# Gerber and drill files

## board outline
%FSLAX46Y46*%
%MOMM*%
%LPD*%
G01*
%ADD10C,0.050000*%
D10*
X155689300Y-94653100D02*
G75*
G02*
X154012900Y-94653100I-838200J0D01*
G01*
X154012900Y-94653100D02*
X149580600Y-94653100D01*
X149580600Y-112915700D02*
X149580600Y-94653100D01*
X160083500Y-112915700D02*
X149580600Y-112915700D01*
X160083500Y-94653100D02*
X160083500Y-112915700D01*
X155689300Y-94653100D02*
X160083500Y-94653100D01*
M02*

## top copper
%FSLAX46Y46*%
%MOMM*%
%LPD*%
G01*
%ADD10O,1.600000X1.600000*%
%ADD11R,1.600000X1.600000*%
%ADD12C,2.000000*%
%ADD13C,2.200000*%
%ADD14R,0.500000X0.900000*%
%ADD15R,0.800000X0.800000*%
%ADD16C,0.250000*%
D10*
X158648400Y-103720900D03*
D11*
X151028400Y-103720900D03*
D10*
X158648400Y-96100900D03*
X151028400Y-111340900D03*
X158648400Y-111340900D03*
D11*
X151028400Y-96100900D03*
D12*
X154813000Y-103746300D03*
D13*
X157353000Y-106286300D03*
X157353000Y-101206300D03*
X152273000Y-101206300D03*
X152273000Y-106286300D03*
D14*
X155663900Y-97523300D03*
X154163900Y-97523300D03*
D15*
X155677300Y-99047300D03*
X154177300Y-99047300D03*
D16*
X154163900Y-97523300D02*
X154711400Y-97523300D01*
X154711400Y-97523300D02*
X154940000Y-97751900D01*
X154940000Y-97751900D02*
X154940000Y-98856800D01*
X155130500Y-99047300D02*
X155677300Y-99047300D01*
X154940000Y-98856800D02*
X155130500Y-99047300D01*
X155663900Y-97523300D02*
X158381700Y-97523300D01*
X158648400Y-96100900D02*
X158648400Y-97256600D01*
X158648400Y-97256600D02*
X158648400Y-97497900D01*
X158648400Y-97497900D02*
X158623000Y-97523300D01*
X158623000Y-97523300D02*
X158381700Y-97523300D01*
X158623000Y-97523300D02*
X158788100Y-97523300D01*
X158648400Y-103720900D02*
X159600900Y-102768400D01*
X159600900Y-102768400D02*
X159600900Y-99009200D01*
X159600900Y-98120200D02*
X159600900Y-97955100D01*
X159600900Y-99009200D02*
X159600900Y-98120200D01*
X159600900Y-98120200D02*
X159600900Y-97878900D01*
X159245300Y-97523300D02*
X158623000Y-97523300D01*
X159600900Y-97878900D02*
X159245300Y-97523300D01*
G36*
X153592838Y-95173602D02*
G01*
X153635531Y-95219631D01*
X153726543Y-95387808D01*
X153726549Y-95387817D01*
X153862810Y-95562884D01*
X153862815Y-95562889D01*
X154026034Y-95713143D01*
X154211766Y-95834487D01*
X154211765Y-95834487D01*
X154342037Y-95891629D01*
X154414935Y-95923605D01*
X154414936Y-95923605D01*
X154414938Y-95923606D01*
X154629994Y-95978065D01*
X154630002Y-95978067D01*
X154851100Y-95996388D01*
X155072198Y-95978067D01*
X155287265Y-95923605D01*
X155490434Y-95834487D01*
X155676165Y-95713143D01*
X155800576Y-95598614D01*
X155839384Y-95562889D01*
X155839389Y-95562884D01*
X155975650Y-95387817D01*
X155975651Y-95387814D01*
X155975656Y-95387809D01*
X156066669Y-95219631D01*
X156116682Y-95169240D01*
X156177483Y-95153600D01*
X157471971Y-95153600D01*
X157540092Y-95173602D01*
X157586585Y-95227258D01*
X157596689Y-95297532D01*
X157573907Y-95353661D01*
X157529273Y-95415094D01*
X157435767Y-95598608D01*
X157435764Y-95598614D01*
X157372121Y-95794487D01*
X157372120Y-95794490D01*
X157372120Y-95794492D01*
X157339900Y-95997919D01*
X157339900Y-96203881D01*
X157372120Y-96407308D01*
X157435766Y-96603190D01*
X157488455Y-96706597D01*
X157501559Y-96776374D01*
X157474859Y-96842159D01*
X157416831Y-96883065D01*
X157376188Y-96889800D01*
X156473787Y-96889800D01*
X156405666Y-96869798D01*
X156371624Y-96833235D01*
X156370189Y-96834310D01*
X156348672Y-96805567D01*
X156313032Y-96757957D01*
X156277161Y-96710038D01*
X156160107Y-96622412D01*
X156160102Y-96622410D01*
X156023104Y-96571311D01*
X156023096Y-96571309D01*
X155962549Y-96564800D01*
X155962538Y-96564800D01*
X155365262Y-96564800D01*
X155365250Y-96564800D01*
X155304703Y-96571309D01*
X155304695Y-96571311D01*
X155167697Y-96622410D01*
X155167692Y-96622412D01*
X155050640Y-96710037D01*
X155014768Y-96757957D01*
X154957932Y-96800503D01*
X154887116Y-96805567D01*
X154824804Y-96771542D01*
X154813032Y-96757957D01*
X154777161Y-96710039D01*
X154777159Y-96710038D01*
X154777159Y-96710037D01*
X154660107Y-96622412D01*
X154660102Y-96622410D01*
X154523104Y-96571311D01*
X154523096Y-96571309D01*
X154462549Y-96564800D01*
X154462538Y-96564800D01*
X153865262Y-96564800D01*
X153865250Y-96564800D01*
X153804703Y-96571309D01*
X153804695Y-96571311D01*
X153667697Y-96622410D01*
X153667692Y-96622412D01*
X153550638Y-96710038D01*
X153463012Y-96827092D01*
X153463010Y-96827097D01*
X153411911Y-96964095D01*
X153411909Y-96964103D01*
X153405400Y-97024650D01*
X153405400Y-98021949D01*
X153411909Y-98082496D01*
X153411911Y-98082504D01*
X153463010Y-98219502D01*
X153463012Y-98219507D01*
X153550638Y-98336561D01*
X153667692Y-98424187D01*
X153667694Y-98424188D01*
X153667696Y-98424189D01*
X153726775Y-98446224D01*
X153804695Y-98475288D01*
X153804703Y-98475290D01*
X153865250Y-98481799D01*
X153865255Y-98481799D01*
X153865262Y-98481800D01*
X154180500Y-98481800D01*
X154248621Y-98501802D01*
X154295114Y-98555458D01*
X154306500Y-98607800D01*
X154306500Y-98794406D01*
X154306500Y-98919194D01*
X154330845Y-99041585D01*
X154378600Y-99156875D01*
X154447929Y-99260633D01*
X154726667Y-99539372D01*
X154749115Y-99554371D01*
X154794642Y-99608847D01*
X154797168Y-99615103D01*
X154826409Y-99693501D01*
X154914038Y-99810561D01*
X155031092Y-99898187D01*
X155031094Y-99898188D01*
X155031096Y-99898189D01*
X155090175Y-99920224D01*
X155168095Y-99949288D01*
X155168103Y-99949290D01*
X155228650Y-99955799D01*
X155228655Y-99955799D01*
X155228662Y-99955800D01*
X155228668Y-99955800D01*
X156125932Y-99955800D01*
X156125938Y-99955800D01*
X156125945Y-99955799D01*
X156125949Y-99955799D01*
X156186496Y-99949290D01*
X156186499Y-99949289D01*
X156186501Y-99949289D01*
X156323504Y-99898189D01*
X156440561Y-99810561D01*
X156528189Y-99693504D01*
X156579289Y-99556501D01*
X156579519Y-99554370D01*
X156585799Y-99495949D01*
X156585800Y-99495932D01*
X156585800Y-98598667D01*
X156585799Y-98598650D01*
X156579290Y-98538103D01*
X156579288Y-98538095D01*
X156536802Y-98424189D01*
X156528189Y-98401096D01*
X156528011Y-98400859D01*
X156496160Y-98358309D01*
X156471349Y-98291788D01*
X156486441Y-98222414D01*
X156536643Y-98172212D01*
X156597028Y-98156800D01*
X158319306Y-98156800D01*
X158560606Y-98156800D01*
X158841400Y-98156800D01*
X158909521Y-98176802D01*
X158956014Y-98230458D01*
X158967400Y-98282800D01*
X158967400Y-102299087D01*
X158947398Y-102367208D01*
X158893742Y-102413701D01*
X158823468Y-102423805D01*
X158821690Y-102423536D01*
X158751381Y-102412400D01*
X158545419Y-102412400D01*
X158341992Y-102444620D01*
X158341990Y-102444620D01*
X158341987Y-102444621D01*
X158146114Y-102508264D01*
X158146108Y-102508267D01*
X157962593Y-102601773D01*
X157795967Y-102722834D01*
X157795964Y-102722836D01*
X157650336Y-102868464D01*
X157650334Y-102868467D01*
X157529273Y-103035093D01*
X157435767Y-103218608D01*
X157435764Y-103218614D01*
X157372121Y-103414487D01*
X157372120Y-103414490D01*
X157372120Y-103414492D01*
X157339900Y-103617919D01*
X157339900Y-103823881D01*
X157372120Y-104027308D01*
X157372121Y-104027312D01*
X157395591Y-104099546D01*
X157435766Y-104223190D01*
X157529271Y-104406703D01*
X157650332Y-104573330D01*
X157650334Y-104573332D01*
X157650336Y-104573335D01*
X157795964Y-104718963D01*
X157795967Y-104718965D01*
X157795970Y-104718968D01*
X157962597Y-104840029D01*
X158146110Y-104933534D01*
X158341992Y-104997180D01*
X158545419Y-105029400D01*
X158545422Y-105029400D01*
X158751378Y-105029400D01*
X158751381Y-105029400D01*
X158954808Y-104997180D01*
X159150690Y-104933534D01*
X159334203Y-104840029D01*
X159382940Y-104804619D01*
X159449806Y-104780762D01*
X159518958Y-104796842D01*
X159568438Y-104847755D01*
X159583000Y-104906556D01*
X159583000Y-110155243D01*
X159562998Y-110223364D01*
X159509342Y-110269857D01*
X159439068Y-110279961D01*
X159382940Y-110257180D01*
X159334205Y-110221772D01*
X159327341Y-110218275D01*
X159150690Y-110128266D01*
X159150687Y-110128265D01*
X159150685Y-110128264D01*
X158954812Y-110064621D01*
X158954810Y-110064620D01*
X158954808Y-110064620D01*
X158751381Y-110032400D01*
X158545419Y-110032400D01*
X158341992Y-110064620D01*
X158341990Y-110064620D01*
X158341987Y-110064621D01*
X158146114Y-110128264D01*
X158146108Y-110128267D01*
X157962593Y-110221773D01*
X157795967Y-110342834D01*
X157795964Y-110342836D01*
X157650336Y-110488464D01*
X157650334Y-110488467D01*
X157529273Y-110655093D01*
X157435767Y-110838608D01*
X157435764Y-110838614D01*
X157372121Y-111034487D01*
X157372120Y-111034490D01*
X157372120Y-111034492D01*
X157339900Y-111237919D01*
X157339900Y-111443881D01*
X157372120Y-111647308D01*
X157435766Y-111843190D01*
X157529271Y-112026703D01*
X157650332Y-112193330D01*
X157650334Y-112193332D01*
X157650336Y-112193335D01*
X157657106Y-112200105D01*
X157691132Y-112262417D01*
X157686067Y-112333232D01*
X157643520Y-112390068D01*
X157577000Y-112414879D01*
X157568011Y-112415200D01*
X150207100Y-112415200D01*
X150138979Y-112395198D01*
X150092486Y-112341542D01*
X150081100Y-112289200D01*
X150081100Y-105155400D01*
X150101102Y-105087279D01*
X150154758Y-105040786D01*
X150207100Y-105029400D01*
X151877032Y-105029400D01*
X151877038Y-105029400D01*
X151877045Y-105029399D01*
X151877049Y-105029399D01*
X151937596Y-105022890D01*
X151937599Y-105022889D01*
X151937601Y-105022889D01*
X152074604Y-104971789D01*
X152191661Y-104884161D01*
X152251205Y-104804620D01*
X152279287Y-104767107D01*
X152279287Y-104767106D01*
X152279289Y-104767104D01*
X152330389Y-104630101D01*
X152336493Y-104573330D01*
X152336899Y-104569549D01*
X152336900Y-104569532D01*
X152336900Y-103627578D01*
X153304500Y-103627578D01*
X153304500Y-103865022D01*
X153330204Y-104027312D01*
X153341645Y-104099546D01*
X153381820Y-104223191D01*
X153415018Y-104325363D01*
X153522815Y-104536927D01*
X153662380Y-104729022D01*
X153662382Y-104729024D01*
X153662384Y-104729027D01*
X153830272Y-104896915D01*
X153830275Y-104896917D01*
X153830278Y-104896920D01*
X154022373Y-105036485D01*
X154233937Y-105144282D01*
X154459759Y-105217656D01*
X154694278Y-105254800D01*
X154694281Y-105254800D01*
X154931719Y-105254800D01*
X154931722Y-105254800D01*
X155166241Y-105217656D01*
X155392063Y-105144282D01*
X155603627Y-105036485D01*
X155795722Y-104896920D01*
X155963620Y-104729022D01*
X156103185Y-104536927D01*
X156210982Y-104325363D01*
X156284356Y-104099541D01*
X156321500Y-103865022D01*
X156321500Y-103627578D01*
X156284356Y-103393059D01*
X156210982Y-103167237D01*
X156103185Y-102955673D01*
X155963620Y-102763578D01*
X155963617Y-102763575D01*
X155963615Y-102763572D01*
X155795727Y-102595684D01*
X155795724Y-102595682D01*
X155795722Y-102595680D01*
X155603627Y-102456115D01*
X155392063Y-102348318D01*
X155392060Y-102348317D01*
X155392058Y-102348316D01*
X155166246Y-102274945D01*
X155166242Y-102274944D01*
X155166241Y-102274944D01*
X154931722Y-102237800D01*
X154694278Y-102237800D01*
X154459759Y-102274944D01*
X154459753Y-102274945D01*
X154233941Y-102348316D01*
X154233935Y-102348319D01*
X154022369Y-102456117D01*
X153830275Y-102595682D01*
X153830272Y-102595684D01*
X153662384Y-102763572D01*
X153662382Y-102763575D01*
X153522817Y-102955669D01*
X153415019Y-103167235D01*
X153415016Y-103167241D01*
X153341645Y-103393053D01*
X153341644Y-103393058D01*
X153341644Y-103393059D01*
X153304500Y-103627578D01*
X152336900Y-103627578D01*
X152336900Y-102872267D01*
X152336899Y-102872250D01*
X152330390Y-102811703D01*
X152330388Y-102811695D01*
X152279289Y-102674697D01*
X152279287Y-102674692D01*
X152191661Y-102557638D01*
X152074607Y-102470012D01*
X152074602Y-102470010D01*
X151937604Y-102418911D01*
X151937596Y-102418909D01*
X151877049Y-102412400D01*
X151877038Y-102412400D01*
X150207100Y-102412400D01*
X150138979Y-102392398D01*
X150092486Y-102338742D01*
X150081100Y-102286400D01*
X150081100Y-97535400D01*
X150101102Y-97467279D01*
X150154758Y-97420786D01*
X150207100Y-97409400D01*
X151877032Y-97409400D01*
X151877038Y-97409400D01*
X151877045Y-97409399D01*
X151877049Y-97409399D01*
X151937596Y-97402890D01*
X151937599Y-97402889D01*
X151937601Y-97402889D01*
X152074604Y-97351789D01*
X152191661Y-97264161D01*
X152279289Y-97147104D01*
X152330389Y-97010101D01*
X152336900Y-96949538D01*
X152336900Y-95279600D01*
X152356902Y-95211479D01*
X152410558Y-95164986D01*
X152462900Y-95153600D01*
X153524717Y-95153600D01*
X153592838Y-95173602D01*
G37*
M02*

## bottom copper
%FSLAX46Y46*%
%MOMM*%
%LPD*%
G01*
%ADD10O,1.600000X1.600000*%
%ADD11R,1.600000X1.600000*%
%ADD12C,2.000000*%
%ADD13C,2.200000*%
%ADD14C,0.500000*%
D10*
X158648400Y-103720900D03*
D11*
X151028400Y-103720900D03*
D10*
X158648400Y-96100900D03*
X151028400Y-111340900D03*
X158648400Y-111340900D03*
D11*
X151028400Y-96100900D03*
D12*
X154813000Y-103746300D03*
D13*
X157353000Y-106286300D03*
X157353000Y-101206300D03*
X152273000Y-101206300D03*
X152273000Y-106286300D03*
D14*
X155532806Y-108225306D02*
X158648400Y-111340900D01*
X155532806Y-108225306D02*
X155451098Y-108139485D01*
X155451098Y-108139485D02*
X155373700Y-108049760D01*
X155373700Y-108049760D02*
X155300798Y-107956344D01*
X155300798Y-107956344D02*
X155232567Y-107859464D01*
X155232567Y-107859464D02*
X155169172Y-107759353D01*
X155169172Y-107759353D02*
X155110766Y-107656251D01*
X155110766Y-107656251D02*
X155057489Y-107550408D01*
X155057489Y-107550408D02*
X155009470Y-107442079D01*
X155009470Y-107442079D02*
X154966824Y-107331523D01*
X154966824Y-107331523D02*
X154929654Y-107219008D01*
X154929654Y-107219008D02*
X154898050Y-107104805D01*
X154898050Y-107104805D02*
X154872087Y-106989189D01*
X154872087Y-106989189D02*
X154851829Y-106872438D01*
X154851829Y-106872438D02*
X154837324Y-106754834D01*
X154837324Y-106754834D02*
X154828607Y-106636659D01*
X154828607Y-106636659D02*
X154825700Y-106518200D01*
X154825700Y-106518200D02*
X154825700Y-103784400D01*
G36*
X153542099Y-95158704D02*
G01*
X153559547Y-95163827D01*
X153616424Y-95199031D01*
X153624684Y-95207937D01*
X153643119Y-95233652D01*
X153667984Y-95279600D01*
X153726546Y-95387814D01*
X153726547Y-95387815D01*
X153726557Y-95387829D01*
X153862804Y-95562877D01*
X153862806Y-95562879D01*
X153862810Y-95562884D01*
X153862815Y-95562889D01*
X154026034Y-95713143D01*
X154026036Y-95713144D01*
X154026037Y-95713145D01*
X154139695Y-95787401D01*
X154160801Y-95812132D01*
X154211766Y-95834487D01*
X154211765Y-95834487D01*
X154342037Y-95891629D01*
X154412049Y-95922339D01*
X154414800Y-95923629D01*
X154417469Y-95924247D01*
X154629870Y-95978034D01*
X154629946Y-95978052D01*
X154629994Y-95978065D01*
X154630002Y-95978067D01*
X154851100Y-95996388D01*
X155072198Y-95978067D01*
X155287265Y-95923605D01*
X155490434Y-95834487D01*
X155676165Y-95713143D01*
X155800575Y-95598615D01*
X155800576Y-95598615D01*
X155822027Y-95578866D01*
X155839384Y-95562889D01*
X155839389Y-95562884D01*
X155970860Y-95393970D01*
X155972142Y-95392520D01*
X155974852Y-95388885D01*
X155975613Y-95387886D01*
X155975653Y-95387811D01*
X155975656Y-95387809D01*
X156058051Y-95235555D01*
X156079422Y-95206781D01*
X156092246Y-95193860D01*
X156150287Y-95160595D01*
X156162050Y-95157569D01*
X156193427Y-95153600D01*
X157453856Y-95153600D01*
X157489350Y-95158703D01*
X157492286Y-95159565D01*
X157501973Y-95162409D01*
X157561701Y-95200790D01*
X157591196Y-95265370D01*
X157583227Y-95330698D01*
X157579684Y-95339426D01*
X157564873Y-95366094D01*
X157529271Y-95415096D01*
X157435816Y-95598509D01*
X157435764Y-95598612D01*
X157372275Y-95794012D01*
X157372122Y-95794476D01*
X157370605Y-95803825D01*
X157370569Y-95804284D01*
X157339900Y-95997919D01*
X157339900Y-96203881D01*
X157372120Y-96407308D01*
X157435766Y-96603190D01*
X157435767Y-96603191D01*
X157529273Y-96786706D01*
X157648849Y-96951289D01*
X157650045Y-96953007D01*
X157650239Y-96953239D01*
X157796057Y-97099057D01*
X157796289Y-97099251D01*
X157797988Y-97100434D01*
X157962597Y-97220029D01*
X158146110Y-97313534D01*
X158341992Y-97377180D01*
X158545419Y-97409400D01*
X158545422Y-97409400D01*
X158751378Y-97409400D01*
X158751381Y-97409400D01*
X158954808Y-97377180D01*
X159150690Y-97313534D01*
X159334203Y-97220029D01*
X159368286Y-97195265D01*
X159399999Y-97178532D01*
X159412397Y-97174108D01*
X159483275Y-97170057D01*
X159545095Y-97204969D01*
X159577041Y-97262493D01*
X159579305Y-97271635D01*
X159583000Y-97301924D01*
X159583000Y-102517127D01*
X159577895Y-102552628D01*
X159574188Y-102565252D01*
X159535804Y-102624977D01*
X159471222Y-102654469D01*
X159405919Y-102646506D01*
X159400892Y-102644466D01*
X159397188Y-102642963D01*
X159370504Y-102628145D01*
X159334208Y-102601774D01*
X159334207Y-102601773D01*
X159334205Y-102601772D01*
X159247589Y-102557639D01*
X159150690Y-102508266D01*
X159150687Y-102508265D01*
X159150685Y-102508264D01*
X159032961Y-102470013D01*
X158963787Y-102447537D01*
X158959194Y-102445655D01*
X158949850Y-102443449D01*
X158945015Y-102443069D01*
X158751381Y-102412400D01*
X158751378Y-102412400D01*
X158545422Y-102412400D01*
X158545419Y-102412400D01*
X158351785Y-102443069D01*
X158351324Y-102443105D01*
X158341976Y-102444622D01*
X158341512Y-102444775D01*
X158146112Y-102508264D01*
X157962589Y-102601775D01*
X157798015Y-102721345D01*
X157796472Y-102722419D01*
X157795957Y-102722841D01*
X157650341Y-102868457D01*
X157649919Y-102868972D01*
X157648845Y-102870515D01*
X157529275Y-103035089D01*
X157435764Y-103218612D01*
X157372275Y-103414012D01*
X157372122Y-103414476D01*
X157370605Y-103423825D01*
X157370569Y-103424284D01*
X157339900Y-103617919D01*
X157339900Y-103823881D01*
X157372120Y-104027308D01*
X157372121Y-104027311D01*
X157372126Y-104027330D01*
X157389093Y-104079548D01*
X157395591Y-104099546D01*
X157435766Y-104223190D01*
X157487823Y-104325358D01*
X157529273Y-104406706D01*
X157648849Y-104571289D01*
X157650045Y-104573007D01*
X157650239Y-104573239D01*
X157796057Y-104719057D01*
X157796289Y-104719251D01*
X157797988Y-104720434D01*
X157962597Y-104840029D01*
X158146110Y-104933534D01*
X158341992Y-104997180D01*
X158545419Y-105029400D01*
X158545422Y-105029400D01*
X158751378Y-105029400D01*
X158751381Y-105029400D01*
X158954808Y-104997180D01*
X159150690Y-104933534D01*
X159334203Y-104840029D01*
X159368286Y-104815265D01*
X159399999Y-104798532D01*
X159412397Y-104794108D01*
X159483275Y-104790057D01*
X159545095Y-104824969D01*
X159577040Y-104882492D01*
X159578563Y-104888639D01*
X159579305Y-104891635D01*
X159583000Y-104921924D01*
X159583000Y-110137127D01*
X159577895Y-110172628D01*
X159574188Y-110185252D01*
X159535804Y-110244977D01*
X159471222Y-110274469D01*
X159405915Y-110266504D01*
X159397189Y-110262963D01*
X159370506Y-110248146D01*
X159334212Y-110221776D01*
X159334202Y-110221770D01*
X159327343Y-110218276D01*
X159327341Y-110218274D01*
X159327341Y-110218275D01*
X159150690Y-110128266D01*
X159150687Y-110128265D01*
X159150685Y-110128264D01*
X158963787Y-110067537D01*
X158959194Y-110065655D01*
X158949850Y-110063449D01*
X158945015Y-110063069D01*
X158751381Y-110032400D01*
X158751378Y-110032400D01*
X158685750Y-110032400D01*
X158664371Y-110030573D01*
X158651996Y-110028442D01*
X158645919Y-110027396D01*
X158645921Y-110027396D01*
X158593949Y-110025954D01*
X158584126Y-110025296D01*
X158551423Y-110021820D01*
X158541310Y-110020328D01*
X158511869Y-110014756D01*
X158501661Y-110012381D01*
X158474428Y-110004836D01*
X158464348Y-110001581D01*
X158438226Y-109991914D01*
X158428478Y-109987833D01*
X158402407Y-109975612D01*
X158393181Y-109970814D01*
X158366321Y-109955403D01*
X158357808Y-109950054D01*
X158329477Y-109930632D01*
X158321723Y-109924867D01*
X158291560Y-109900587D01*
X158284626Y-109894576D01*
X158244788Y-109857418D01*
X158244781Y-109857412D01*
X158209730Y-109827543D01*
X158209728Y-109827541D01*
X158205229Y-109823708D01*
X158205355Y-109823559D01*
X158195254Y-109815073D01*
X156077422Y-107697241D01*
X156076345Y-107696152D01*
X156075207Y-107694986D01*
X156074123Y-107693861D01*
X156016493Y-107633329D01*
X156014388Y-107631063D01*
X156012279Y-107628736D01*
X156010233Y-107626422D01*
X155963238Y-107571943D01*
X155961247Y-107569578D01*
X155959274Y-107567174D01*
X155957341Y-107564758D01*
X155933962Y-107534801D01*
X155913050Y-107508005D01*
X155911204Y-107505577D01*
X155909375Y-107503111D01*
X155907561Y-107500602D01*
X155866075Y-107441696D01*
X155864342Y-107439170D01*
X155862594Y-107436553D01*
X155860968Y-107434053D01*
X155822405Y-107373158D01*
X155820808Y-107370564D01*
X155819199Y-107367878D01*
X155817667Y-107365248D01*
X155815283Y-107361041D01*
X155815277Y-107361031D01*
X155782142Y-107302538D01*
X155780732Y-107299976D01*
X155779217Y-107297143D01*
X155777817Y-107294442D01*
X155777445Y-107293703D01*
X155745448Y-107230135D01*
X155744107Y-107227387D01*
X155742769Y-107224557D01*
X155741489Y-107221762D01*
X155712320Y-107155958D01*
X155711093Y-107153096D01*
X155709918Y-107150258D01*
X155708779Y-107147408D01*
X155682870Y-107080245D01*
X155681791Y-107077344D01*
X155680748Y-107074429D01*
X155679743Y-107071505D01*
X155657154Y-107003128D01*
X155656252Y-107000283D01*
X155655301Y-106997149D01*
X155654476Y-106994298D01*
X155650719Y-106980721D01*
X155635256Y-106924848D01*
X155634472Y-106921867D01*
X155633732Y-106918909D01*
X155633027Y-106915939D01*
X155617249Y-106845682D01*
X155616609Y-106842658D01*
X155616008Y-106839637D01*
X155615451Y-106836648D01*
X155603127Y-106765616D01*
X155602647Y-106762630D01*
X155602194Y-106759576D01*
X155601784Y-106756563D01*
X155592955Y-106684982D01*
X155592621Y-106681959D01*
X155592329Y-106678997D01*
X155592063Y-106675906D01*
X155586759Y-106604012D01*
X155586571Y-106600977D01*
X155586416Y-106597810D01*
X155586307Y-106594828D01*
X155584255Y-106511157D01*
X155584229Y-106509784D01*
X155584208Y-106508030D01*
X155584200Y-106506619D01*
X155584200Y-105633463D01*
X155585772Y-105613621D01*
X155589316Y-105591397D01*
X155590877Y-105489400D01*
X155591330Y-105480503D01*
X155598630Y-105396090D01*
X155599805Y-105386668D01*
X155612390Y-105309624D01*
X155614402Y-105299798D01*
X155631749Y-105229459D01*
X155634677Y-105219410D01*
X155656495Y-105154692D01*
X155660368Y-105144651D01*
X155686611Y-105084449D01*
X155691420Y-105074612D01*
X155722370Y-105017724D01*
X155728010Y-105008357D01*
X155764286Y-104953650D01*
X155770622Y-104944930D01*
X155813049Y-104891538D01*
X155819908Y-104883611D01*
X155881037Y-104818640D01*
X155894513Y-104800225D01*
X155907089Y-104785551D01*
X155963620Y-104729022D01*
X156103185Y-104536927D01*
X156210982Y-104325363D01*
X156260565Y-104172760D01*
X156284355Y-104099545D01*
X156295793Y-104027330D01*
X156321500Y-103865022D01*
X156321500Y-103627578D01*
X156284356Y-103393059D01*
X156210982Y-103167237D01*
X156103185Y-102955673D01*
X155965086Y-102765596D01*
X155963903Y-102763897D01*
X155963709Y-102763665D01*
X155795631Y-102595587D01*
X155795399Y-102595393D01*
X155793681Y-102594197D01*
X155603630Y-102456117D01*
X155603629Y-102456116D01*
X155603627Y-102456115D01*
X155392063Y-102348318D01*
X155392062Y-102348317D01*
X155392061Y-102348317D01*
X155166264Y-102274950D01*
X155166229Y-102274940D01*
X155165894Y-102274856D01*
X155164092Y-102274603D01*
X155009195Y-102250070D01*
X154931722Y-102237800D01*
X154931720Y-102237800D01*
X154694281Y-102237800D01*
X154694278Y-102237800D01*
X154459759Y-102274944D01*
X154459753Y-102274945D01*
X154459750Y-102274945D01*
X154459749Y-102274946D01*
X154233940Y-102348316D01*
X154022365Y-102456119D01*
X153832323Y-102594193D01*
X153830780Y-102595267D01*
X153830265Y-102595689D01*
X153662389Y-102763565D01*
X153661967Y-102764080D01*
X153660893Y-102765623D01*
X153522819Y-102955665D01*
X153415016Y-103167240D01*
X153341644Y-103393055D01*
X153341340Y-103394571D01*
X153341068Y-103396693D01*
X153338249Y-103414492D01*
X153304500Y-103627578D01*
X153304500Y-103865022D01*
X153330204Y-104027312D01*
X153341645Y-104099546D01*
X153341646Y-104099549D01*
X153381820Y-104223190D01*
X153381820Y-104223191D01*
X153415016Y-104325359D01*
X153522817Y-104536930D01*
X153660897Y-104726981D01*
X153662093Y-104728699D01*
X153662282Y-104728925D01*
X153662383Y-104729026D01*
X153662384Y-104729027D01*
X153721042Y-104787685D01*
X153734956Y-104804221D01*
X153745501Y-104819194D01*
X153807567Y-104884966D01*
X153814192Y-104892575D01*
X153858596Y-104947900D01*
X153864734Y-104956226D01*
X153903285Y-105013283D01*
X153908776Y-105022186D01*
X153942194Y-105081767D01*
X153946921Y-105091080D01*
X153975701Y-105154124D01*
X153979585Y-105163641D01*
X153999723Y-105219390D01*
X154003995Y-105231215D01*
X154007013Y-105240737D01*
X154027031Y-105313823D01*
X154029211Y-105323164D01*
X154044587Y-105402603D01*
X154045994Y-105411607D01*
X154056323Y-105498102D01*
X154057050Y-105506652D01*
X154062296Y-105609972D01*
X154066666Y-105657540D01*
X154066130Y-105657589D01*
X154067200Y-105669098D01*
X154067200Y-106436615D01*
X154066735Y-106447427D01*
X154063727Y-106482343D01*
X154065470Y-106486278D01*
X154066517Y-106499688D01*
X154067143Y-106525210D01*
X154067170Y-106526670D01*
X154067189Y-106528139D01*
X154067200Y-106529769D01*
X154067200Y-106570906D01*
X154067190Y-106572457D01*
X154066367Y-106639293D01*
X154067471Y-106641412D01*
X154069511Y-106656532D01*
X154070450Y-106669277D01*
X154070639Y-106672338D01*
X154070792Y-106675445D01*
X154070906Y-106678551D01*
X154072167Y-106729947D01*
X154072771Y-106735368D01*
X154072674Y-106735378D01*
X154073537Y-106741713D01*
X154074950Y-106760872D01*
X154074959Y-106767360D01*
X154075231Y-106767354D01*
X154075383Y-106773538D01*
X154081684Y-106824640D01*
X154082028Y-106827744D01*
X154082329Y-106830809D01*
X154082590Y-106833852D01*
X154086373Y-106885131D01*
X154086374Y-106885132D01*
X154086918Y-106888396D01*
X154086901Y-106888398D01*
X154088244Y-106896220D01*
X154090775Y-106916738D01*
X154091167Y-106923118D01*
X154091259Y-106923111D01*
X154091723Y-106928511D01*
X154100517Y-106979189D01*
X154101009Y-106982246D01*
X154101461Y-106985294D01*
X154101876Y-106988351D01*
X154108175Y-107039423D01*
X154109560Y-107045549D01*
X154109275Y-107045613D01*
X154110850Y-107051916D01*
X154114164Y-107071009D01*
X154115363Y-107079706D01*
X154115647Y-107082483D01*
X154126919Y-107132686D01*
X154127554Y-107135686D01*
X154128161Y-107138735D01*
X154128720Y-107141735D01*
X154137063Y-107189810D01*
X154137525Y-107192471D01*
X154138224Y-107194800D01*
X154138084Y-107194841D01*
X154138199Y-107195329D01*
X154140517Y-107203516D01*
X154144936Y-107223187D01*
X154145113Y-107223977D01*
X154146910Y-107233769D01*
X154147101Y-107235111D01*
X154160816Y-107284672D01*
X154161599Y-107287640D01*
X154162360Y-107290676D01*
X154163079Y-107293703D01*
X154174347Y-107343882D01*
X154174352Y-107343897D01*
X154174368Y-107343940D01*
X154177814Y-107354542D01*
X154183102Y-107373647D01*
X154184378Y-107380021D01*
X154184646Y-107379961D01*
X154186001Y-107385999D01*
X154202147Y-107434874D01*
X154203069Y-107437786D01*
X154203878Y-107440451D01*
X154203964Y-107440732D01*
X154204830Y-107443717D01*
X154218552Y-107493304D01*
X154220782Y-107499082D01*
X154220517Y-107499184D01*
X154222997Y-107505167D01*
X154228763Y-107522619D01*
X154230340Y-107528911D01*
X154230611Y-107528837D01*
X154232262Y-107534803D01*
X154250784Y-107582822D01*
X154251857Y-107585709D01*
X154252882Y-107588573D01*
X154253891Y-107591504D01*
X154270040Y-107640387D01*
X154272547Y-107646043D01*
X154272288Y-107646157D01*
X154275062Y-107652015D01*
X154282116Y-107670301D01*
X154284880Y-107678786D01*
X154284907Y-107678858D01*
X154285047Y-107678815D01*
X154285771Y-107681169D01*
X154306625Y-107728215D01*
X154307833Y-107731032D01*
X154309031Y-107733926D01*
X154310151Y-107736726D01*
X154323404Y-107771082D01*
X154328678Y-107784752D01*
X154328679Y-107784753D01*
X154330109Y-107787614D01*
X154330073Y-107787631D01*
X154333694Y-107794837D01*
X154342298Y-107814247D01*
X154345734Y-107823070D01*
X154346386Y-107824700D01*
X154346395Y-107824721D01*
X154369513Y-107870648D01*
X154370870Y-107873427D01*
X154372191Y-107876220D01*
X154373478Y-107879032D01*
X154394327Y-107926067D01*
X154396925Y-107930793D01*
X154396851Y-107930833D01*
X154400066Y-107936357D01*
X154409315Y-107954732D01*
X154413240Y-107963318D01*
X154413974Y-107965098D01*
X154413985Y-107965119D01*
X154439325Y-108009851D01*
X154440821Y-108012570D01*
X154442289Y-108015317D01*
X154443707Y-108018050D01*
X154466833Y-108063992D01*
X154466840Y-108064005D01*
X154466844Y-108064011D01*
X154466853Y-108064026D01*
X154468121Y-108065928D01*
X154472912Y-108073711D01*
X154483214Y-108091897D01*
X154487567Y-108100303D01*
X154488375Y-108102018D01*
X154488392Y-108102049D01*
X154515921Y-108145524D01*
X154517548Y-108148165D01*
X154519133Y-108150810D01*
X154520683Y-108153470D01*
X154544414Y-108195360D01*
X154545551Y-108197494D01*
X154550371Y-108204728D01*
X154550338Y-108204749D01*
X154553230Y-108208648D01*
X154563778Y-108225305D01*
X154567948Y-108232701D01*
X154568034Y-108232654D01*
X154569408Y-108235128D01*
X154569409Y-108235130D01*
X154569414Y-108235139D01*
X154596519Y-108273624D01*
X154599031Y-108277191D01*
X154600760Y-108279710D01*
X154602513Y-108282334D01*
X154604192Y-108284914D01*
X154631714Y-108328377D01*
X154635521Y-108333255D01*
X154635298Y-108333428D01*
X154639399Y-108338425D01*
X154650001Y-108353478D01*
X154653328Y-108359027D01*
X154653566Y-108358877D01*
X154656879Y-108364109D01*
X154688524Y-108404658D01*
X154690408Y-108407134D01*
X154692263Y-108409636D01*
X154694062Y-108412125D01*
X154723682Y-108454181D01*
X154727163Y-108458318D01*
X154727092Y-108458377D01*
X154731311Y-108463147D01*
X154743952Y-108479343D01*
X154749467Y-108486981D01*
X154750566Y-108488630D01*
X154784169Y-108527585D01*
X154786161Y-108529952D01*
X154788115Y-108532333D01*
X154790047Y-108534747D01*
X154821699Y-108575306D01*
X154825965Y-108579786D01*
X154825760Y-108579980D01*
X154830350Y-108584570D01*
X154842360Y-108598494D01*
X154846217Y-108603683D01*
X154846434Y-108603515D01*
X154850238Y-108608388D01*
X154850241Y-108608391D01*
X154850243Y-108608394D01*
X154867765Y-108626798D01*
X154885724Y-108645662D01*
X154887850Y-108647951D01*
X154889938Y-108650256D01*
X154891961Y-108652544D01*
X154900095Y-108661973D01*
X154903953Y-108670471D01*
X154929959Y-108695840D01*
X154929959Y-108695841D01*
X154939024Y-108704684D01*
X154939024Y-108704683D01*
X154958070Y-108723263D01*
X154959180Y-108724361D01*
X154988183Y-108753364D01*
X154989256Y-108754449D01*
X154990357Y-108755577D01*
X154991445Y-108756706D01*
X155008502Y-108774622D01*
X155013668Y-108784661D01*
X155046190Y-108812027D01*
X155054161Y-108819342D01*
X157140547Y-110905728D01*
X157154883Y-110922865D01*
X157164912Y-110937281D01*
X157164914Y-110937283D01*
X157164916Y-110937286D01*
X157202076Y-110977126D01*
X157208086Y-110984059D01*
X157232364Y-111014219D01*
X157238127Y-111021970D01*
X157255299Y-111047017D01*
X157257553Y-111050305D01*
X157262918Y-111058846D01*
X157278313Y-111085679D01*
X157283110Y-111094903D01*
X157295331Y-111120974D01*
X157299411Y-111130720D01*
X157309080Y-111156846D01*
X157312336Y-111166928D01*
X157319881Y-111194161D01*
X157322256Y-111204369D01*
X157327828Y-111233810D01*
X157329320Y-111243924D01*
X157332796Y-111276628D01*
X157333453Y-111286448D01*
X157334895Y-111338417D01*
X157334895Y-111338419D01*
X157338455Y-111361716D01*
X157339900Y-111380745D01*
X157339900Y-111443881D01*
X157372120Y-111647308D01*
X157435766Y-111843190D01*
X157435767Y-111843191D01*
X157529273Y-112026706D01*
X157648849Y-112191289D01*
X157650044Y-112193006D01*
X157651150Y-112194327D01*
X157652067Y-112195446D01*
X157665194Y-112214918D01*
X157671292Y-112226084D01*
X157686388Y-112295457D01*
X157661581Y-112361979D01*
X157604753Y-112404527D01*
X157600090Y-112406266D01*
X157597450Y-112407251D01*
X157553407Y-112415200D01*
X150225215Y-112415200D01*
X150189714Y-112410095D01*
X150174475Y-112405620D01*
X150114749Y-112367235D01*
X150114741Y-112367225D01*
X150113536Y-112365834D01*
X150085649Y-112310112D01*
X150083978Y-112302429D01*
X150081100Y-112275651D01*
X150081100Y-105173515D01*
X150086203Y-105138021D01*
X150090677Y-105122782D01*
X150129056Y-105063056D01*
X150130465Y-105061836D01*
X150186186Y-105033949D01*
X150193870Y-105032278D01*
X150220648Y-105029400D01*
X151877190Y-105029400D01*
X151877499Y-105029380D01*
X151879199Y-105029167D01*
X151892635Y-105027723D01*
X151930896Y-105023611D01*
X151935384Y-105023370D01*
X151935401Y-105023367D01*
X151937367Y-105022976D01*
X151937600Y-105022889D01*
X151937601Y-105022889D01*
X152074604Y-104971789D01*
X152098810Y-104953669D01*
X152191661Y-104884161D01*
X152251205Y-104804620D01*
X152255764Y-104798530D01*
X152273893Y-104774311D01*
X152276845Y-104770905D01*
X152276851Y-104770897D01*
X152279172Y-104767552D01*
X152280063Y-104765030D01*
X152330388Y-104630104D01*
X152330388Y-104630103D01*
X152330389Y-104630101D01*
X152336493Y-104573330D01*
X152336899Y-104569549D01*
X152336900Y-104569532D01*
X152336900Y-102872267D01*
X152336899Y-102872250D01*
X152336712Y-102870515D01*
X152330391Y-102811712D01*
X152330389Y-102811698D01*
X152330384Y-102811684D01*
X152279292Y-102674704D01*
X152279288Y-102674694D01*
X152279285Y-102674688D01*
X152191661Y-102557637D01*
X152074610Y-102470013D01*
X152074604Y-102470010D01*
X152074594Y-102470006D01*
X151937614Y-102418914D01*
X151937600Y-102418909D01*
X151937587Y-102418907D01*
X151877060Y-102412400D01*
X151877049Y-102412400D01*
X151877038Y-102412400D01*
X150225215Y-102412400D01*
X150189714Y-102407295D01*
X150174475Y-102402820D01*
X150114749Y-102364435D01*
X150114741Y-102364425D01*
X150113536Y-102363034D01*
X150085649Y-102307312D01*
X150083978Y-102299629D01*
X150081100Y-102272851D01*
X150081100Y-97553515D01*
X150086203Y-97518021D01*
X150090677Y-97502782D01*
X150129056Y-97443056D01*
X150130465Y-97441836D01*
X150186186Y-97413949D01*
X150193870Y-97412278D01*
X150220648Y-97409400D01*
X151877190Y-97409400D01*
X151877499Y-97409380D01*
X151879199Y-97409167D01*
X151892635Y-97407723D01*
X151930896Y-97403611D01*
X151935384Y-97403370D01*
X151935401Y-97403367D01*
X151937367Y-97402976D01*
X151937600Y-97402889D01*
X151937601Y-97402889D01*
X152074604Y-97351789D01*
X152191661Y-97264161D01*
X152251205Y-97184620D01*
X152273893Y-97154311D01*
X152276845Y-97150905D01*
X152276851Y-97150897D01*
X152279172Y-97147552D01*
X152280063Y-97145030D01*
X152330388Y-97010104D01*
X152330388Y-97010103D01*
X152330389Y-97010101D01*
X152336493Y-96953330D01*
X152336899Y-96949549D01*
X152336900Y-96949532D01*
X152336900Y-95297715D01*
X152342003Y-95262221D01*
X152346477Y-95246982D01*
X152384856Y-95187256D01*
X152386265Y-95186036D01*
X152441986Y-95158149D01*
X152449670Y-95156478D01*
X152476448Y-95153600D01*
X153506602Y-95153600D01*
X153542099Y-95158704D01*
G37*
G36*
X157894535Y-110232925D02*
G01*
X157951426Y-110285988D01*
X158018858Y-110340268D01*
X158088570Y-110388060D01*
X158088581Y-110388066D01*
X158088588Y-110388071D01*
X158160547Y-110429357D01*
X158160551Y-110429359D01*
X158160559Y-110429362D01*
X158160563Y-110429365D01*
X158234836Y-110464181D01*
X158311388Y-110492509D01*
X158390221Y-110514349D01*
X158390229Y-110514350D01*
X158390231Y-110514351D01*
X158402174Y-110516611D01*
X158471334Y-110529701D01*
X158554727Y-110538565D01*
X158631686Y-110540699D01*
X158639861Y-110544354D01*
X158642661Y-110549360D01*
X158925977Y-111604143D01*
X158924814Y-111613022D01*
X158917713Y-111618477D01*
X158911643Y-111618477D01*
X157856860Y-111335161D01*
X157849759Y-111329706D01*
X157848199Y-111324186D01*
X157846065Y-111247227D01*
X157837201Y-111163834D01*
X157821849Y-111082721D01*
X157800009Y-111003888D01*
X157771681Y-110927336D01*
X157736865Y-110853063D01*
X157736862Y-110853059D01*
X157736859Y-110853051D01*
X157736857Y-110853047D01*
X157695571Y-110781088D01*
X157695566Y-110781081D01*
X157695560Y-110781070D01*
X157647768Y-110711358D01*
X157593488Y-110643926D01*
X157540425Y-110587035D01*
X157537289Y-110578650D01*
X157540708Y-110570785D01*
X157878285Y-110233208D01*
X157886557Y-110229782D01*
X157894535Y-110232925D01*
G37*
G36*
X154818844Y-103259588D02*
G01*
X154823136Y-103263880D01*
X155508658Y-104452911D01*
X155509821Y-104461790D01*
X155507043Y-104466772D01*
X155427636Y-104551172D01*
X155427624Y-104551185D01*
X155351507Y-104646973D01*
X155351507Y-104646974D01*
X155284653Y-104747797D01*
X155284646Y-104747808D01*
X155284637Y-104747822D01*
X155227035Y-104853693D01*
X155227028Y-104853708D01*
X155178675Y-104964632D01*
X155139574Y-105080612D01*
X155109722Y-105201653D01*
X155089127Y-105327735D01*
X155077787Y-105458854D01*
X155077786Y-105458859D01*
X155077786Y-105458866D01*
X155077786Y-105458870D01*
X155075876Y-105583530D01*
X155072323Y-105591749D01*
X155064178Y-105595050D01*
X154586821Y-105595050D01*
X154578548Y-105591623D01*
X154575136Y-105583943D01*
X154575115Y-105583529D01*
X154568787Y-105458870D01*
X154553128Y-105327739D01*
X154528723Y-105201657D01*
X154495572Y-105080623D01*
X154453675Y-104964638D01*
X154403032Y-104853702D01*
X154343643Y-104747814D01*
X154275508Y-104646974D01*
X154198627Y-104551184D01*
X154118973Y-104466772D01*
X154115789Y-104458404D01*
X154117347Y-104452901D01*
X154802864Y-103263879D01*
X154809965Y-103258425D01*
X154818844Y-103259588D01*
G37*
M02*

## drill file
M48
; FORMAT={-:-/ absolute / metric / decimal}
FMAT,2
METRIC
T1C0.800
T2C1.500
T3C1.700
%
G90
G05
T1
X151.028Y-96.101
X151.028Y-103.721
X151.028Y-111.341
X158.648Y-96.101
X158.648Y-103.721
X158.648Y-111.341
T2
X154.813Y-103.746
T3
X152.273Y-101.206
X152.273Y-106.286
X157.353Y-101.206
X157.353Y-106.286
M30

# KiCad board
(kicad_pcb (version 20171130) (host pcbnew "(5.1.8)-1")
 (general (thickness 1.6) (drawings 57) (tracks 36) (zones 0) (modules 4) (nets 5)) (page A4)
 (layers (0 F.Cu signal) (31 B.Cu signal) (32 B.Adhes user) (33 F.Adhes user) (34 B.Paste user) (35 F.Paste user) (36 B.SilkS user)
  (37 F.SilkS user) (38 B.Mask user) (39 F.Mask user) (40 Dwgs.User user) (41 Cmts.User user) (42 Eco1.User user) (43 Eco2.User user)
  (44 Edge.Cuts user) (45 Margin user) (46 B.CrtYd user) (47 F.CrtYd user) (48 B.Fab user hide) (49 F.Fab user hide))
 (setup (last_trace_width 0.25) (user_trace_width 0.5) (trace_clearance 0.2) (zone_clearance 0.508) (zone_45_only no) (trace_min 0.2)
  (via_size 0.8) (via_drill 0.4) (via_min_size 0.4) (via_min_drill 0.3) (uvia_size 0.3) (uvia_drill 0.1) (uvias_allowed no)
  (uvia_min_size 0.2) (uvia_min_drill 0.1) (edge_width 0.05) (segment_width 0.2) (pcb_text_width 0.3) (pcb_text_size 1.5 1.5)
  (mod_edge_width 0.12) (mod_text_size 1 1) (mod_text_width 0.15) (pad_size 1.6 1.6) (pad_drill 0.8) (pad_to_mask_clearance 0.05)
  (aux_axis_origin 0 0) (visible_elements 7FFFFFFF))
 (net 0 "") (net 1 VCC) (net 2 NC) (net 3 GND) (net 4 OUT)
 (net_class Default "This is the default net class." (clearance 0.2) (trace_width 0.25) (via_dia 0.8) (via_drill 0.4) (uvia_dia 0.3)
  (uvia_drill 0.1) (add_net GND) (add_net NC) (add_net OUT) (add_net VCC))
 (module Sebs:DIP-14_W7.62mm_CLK (layer F.Cu) (at 151.0284 96.1009)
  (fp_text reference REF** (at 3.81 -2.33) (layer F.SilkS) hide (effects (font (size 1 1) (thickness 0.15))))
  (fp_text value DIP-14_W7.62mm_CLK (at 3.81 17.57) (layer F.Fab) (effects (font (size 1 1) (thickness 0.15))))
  (pad 11 thru_hole oval (at 7.62 7.62) (size 1.6 1.6) (drill 0.8) (layers *.Cu *.Mask) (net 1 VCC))
  (pad 4 thru_hole rect (at 0 7.62) (size 1.6 1.6) (drill 0.8) (layers *.Cu *.Mask) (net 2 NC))
  (pad 14 thru_hole oval (at 7.62 0) (size 1.6 1.6) (drill 0.8) (layers *.Cu *.Mask) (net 1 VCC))
  (pad 7 thru_hole oval (at 0 15.24) (size 1.6 1.6) (drill 0.8) (layers *.Cu *.Mask) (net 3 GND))
  (pad 8 thru_hole oval (at 7.62 15.24) (size 1.6 1.6) (drill 0.8) (layers *.Cu *.Mask) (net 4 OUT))
  (pad 1 thru_hole rect (at 0 0) (size 1.6 1.6) (drill 0.8) (layers *.Cu *.Mask) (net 2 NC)))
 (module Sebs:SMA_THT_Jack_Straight (layer F.Cu) (at 154.813 103.7463)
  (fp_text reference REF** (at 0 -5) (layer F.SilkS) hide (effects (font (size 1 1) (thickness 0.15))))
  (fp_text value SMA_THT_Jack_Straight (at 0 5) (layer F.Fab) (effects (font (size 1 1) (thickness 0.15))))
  (pad 1 thru_hole circle (at 0 0) (size 2 2) (drill 1.5) (layers *.Cu *.Mask) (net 4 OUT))
  (pad 2 thru_hole circle (at 2.54 2.54) (size 2.2 2.2) (drill 1.7) (layers *.Cu *.Mask) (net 3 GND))
  (pad 2 thru_hole circle (at 2.54 -2.54) (size 2.2 2.2) (drill 1.7) (layers *.Cu *.Mask) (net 3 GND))
  (pad 2 thru_hole circle (at -2.54 -2.54) (size 2.2 2.2) (drill 1.7) (layers *.Cu *.Mask) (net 3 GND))
  (pad 2 thru_hole circle (at -2.54 2.54) (size 2.2 2.2) (drill 1.7) (layers *.Cu *.Mask) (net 3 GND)))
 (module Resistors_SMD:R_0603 (layer F.Cu) (at 154.9139 97.5233 180)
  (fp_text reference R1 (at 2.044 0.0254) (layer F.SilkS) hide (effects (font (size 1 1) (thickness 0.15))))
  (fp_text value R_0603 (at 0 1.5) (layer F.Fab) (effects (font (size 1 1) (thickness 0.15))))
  (pad 1 smd rect (at -0.75 0 180) (size 0.5 0.9) (layers F.Cu F.Paste F.Mask) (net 1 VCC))
  (pad 2 smd rect (at 0.75 0 180) (size 0.5 0.9) (layers F.Cu F.Paste F.Mask)))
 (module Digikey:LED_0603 (layer F.Cu) (at 154.9273 99.0473)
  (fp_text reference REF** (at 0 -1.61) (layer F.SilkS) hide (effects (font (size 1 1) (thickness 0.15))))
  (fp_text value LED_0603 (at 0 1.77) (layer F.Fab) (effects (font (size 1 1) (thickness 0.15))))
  (pad 2 smd rect (at 0.75 0) (size 0.8 0.8) (layers F.Cu F.Paste F.Mask))
  (pad 1 smd rect (at -0.75 0) (size 0.8 0.8) (layers F.Cu F.Paste F.Mask) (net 3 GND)))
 (gr_arc (start 154.8511 94.6531) (end 154.0129 94.6531) (angle -180) (layer Edge.Cuts) (width 0.05))
 (gr_line (start 154.0129 94.6531) (end 149.5806 94.6531) (layer Edge.Cuts) (width 0.05))
 (gr_line (start 149.5806 112.9157) (end 149.5806 94.6531) (layer Edge.Cuts) (width 0.05))
 (gr_line (start 160.0835 112.9157) (end 149.5806 112.9157) (layer Edge.Cuts) (width 0.05))
 (gr_line (start 160.0835 94.6531) (end 160.0835 112.9157) (layer Edge.Cuts) (width 0.05))
 (gr_line (start 155.6893 94.6531) (end 160.0835 94.6531) (layer Edge.Cuts) (width 0.05))
 (segment (start 154.1639 97.5233) (end 154.7114 97.5233) (width 0.25) (layer F.Cu) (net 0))
 (segment (start 154.7114 97.5233) (end 154.94 97.7519) (width 0.25) (layer F.Cu) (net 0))
 (segment (start 154.94 97.7519) (end 154.94 98.8568) (width 0.25) (layer F.Cu) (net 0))
 (segment (start 155.1305 99.0473) (end 155.6773 99.0473) (width 0.25) (layer F.Cu) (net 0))
 (segment (start 154.94 98.8568) (end 155.1305 99.0473) (width 0.25) (layer F.Cu) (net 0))
 (segment (start 155.532806 108.225306) (end 158.6484 111.3409) (width 0.5) (layer B.Cu) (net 4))
 (segment (start 155.532806 108.225306) (end 155.451098 108.139485) (width 0.5) (layer B.Cu) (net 4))
 (segment (start 155.451098 108.139485) (end 155.3737 108.04976) (width 0.5) (layer B.Cu) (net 4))
 (segment (start 155.3737 108.04976) (end 155.300798 107.956344) (width 0.5) (layer B.Cu) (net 4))
 (segment (start 155.300798 107.956344) (end 155.232567 107.859464) (width 0.5) (layer B.Cu) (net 4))
 (segment (start 155.232567 107.859464) (end 155.169172 107.759353) (width 0.5) (layer B.Cu) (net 4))
 (segment (start 155.169172 107.759353) (end 155.110766 107.656251) (width 0.5) (layer B.Cu) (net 4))
 (segment (start 155.110766 107.656251) (end 155.057489 107.550408) (width 0.5) (layer B.Cu) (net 4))
 (segment (start 155.057489 107.550408) (end 155.00947 107.442079) (width 0.5) (layer B.Cu) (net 4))
 (segment (start 155.00947 107.442079) (end 154.966824 107.331523) (width 0.5) (layer B.Cu) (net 4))
 (segment (start 154.966824 107.331523) (end 154.929654 107.219008) (width 0.5) (layer B.Cu) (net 4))
 (segment (start 154.929654 107.219008) (end 154.89805 107.104805) (width 0.5) (layer B.Cu) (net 4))
 (segment (start 154.89805 107.104805) (end 154.872087 106.989189) (width 0.5) (layer B.Cu) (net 4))
 (segment (start 154.872087 106.989189) (end 154.851829 106.872438) (width 0.5) (layer B.Cu) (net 4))
 (segment (start 154.851829 106.872438) (end 154.837324 106.754834) (width 0.5) (layer B.Cu) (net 4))
 (segment (start 154.837324 106.754834) (end 154.828607 106.636659) (width 0.5) (layer B.Cu) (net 4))
 (segment (start 154.828607 106.636659) (end 154.8257 106.5182) (width 0.5) (layer B.Cu) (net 4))
 (segment (start 154.8257 106.5182) (end 154.8257 103.7844) (width 0.5) (layer B.Cu) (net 4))
 (segment (start 155.6639 97.5233) (end 158.3817 97.5233) (width 0.25) (layer F.Cu) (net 1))
 (segment (start 158.6484 96.1009) (end 158.6484 97.2566) (width 0.25) (layer F.Cu) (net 1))
 (segment (start 158.6484 97.2566) (end 158.6484 97.4979) (width 0.25) (layer F.Cu) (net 1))
 (segment (start 158.6484 97.4979) (end 158.623 97.5233) (width 0.25) (layer F.Cu) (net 1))
 (segment (start 158.623 97.5233) (end 158.3817 97.5233) (width 0.25) (layer F.Cu) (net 1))
 (segment (start 158.623 97.5233) (end 158.7881 97.5233) (width 0.25) (layer F.Cu) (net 1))
 (segment (start 158.6484 103.7209) (end 159.6009 102.7684) (width 0.25) (layer F.Cu) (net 1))
 (segment (start 159.6009 102.7684) (end 159.6009 99.0092) (width 0.25) (layer F.Cu) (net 1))
 (segment (start 159.6009 98.1202) (end 159.6009 97.9551) (width 0.25) (layer F.Cu) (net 1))
 (segment (start 159.6009 99.0092) (end 159.6009 98.1202) (width 0.25) (layer F.Cu) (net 1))
 (segment (start 159.6009 98.1202) (end 159.6009 97.8789) (width 0.25) (layer F.Cu) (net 1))
 (segment (start 159.2453 97.5233) (end 158.623 97.5233) (width 0.25) (layer F.Cu) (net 1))
 (segment (start 159.6009 97.8789) (end 159.2453 97.5233) (width 0.25) (layer F.Cu) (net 1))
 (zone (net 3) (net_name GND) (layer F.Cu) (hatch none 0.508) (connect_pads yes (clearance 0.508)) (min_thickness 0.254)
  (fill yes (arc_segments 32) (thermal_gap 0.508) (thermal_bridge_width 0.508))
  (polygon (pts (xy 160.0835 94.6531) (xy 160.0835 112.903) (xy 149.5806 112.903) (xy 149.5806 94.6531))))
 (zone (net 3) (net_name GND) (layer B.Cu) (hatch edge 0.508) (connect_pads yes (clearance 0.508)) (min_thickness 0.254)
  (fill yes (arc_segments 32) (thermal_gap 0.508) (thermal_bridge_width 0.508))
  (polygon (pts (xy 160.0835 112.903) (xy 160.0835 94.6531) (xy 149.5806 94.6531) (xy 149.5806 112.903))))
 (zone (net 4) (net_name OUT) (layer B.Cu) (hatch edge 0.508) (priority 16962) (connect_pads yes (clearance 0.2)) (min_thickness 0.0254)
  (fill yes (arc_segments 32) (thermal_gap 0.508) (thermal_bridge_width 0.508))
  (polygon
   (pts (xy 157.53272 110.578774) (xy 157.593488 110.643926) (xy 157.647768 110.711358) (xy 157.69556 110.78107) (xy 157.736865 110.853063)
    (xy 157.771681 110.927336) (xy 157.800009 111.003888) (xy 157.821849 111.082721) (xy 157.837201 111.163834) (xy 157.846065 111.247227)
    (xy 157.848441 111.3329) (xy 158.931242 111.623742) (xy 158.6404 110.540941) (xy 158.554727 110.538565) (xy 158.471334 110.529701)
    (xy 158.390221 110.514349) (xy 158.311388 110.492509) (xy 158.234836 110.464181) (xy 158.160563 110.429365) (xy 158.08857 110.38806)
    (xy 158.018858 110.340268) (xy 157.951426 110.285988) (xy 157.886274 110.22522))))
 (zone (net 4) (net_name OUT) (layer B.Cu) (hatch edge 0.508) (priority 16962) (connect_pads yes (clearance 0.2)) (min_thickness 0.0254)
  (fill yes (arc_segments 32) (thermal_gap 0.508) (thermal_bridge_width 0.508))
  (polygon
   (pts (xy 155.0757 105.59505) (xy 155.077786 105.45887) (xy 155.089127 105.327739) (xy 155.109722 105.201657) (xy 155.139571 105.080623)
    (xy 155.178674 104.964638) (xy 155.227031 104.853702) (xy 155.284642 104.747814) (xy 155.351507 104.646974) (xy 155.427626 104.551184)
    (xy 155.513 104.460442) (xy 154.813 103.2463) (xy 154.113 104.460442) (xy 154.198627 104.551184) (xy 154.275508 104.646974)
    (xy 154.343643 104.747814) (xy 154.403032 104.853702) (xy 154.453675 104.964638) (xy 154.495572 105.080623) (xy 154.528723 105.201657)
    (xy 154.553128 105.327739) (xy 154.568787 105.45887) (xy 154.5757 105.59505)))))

